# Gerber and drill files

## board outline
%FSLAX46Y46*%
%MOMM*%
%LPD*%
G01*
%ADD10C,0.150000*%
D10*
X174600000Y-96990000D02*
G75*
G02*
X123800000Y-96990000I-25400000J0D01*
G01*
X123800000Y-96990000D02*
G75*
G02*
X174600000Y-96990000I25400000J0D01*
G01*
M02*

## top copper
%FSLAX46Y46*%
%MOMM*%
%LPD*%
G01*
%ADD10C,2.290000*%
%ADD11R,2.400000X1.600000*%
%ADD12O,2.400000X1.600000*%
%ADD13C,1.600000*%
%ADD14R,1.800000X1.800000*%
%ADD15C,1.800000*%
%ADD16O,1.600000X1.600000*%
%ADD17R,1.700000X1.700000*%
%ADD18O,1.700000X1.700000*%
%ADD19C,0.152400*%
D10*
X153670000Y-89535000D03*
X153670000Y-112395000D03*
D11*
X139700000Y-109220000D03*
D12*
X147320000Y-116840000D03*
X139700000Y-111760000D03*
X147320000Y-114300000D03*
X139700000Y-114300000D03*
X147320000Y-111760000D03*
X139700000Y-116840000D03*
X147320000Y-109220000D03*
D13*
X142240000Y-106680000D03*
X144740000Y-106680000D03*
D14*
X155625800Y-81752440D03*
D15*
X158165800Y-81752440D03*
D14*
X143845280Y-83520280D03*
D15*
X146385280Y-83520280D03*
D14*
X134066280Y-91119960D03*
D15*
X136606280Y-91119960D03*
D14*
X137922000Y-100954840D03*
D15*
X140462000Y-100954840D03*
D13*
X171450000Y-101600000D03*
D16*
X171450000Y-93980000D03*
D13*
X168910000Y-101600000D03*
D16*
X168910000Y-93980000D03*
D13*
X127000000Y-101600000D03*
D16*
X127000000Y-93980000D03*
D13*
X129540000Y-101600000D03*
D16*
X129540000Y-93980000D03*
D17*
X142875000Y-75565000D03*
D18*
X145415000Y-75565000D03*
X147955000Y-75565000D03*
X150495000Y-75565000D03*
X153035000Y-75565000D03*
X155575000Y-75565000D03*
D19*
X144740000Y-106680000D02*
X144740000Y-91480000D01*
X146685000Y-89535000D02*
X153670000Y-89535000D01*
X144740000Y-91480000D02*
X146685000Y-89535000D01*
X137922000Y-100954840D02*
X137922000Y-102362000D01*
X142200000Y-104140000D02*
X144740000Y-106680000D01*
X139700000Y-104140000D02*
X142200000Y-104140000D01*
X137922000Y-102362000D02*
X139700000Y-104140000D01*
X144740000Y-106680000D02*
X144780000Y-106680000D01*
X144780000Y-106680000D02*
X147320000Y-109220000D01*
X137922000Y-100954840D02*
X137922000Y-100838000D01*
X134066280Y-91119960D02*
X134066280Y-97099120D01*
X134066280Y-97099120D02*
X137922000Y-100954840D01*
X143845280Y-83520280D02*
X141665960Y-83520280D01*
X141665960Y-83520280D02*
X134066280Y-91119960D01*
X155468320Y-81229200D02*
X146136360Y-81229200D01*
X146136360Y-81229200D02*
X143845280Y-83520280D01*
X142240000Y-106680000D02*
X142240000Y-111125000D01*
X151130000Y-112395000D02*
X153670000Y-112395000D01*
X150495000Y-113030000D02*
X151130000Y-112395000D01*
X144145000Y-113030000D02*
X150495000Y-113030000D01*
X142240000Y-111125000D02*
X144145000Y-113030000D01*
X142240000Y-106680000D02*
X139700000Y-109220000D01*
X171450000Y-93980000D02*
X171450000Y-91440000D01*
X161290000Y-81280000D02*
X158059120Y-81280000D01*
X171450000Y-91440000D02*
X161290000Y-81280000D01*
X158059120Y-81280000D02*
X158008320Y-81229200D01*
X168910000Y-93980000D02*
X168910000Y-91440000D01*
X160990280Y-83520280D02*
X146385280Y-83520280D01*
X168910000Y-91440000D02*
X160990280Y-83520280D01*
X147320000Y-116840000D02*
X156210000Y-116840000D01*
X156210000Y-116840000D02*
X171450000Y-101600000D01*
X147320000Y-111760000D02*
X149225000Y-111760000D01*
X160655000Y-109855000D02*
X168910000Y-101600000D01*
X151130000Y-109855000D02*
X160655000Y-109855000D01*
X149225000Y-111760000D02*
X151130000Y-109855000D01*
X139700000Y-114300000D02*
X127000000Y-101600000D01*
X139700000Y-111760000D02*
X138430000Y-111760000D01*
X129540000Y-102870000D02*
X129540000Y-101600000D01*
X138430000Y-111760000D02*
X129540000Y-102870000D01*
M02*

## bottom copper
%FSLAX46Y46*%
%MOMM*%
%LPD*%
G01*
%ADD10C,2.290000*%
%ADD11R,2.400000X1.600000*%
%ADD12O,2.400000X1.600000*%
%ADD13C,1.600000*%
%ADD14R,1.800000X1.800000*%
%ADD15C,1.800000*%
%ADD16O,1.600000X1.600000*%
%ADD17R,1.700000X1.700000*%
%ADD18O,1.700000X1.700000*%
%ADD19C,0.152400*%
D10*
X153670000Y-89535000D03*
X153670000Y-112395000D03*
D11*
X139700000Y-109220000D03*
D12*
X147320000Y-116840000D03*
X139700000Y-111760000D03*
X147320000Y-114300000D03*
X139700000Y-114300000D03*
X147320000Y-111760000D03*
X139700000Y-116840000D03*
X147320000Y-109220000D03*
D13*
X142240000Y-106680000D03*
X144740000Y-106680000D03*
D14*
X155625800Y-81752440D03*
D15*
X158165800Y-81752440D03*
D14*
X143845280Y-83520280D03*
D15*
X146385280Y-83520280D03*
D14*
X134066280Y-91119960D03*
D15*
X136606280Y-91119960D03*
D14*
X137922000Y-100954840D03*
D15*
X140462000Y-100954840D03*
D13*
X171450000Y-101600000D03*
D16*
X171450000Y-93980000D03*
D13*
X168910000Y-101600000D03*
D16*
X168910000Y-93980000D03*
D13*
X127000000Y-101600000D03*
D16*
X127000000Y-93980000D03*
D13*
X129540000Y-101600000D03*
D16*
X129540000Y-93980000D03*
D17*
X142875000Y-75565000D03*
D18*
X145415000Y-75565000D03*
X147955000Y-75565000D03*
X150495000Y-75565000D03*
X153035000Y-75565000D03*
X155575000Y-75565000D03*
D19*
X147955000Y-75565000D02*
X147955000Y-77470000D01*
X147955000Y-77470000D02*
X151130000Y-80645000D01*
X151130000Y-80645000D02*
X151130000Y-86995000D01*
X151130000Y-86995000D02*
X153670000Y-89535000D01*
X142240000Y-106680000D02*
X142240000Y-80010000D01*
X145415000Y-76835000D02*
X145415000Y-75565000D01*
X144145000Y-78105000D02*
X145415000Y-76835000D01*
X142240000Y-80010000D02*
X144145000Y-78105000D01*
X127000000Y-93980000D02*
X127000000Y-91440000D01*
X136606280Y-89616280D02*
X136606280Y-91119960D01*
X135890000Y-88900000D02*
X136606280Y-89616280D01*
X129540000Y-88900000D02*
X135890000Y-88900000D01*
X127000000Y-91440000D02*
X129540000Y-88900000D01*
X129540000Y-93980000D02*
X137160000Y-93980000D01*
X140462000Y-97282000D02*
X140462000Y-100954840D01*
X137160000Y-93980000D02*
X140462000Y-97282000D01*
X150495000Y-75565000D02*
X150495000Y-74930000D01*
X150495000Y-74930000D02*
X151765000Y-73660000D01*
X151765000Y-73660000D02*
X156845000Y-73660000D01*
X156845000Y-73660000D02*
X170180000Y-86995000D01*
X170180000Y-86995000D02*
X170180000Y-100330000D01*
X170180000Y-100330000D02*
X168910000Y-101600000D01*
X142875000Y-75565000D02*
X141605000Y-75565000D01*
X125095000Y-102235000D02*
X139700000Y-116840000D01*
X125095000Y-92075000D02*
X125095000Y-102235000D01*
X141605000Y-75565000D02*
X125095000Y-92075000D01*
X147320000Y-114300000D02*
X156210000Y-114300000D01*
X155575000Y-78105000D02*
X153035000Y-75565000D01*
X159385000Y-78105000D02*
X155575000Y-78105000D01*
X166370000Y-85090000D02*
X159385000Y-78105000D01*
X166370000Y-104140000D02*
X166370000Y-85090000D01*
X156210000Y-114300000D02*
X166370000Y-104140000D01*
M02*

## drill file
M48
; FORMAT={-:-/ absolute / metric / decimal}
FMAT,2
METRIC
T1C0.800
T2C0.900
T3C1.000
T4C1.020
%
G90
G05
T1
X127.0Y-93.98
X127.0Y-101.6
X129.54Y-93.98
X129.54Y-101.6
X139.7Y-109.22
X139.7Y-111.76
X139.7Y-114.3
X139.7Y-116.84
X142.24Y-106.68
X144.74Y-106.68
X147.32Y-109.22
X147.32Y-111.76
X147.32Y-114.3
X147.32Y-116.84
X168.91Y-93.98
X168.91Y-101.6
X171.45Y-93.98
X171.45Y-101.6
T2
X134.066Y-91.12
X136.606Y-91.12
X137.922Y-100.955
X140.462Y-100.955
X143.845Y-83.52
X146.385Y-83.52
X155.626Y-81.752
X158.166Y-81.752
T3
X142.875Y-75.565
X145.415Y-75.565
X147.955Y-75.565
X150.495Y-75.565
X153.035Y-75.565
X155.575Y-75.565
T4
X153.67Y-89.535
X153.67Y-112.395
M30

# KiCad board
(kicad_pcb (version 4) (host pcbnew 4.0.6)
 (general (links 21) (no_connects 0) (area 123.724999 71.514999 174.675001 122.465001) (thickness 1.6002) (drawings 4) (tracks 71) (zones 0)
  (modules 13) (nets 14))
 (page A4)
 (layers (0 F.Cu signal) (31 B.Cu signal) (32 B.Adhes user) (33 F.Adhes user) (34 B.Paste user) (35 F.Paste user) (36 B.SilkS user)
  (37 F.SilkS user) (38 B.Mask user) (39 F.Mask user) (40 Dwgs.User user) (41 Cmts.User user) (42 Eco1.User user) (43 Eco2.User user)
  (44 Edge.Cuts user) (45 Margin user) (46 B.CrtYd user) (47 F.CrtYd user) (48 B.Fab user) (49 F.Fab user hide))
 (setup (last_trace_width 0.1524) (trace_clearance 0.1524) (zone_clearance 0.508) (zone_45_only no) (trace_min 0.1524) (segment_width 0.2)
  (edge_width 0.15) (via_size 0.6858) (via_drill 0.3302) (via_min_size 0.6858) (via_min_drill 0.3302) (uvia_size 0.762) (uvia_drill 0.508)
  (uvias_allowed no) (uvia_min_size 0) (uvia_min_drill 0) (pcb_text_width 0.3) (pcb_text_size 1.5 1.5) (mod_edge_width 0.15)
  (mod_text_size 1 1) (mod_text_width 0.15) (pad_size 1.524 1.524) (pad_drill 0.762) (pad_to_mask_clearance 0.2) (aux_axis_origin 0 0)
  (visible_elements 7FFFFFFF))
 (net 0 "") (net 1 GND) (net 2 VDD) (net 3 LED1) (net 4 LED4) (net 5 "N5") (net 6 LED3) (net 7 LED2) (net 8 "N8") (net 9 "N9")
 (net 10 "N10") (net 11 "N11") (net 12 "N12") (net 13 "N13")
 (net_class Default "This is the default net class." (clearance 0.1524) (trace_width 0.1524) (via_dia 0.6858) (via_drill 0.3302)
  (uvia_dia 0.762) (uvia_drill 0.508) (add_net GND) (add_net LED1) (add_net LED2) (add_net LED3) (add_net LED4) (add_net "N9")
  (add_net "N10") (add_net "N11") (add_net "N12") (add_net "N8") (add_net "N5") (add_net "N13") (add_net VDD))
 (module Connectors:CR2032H (layer B.Cu) (at 153.67 112.395 270)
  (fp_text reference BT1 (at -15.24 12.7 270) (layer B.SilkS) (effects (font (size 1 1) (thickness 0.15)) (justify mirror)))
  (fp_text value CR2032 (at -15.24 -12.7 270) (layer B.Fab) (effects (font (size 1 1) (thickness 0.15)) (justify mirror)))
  (pad 2 thru_hole circle (at -22.86 0 270) (size 2.29 2.29) (drill 1.02) (layers *.Cu *.Mask) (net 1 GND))
  (pad 1 thru_hole circle (at 0 0 270) (size 2.29 2.29) (drill 1.02) (layers *.Cu *.Mask) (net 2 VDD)))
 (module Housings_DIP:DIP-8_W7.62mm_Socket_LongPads (layer F.Cu) (at 139.7 109.22)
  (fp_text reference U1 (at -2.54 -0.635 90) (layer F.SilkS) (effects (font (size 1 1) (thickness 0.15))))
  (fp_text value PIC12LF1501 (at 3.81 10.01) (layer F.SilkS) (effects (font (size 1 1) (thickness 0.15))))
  (pad 1 thru_hole rect (at 0 0) (size 2.4 1.6) (drill 0.8) (layers *.Cu *.Mask) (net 2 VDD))
  (pad 5 thru_hole oval (at 7.62 7.62) (size 2.4 1.6) (drill 0.8) (layers *.Cu *.Mask) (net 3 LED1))
  (pad 2 thru_hole oval (at 0 2.54) (size 2.4 1.6) (drill 0.8) (layers *.Cu *.Mask) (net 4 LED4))
  (pad 6 thru_hole oval (at 7.62 5.08) (size 2.4 1.6) (drill 0.8) (layers *.Cu *.Mask) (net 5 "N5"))
  (pad 3 thru_hole oval (at 0 5.08) (size 2.4 1.6) (drill 0.8) (layers *.Cu *.Mask) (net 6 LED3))
  (pad 7 thru_hole oval (at 7.62 2.54) (size 2.4 1.6) (drill 0.8) (layers *.Cu *.Mask) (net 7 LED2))
  (pad 4 thru_hole oval (at 0 7.62) (size 2.4 1.6) (drill 0.8) (layers *.Cu *.Mask) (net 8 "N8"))
  (pad 8 thru_hole oval (at 7.62 0) (size 2.4 1.6) (drill 0.8) (layers *.Cu *.Mask) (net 1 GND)))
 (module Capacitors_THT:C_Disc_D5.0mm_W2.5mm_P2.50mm (layer F.Cu) (at 142.24 106.68)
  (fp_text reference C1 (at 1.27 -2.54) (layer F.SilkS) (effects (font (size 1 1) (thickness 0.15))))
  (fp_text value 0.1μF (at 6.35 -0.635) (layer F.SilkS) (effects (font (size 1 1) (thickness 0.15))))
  (pad 1 thru_hole circle (at 0 0) (size 1.6 1.6) (drill 0.8) (layers *.Cu *.Mask) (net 2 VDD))
  (pad 2 thru_hole circle (at 2.5 0) (size 1.6 1.6) (drill 0.8) (layers *.Cu *.Mask) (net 1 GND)))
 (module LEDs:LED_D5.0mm (layer F.Cu) (at 155.6258 81.75244)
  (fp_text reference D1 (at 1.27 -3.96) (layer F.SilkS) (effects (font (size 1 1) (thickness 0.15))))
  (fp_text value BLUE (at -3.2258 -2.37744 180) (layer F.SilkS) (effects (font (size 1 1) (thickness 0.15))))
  (pad 1 thru_hole rect (at 0 0) (size 1.8 1.8) (drill 0.9) (layers *.Cu *.Mask) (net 1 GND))
  (pad 2 thru_hole circle (at 2.54 0) (size 1.8 1.8) (drill 0.9) (layers *.Cu *.Mask) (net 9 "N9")))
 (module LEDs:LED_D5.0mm (layer F.Cu) (at 143.84528 83.52028)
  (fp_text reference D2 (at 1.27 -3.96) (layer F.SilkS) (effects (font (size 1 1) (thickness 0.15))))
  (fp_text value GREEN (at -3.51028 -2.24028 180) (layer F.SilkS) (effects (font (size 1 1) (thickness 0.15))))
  (pad 1 thru_hole rect (at 0 0) (size 1.8 1.8) (drill 0.9) (layers *.Cu *.Mask) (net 1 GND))
  (pad 2 thru_hole circle (at 2.54 0) (size 1.8 1.8) (drill 0.9) (layers *.Cu *.Mask) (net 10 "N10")))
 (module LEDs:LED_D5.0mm (layer F.Cu) (at 134.06628 91.11996)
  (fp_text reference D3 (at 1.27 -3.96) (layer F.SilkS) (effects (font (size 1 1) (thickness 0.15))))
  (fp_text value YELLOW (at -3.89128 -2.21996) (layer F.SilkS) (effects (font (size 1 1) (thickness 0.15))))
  (pad 1 thru_hole rect (at 0 0) (size 1.8 1.8) (drill 0.9) (layers *.Cu *.Mask) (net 1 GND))
  (pad 2 thru_hole circle (at 2.54 0) (size 1.8 1.8) (drill 0.9) (layers *.Cu *.Mask) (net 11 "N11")))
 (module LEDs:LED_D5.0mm (layer F.Cu) (at 137.922 100.95484)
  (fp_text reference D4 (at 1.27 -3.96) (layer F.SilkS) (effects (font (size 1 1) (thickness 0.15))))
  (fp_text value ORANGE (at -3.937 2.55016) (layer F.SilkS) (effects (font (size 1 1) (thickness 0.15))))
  (pad 1 thru_hole rect (at 0 0) (size 1.8 1.8) (drill 0.9) (layers *.Cu *.Mask) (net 1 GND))
  (pad 2 thru_hole circle (at 2.54 0) (size 1.8 1.8) (drill 0.9) (layers *.Cu *.Mask) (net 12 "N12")))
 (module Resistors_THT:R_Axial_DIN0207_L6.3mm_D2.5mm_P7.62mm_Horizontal (layer F.Cu) (at 171.45 101.6 90)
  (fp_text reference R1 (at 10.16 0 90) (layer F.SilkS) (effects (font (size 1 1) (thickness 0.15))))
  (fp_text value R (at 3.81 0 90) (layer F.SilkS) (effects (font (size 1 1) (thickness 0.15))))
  (pad 1 thru_hole circle (at 0 0 90) (size 1.6 1.6) (drill 0.8) (layers *.Cu *.Mask) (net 3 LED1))
  (pad 2 thru_hole oval (at 7.62 0 90) (size 1.6 1.6) (drill 0.8) (layers *.Cu *.Mask) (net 9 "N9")))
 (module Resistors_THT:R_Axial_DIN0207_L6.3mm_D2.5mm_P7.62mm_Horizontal (layer F.Cu) (at 168.91 101.6 90)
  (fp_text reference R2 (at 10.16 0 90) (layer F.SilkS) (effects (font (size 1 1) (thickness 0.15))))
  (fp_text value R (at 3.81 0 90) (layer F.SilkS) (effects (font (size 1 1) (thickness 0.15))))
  (pad 1 thru_hole circle (at 0 0 90) (size 1.6 1.6) (drill 0.8) (layers *.Cu *.Mask) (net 7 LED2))
  (pad 2 thru_hole oval (at 7.62 0 90) (size 1.6 1.6) (drill 0.8) (layers *.Cu *.Mask) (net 10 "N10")))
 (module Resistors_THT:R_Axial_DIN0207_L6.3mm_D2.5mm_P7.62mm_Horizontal (layer F.Cu) (at 127 101.6 90)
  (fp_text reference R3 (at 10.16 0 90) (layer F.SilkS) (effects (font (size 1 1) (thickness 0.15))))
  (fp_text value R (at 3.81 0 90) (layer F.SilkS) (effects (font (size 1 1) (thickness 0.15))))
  (pad 1 thru_hole circle (at 0 0 90) (size 1.6 1.6) (drill 0.8) (layers *.Cu *.Mask) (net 6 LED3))
  (pad 2 thru_hole oval (at 7.62 0 90) (size 1.6 1.6) (drill 0.8) (layers *.Cu *.Mask) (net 11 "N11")))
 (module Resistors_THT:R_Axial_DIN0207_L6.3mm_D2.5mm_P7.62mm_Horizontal (layer F.Cu) (at 129.54 101.6 90)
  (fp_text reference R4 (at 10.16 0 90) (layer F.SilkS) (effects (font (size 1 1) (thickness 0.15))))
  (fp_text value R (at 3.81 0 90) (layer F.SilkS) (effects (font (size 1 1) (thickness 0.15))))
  (pad 1 thru_hole circle (at 0 0 90) (size 1.6 1.6) (drill 0.8) (layers *.Cu *.Mask) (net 4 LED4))
  (pad 2 thru_hole oval (at 7.62 0 90) (size 1.6 1.6) (drill 0.8) (layers *.Cu *.Mask) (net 12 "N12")))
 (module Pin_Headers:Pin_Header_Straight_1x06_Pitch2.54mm (layer F.Cu) (at 142.875 75.565 90)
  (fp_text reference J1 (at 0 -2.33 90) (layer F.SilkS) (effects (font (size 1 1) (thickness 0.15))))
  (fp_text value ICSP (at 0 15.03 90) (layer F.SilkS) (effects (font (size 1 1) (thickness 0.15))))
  (pad 1 thru_hole rect (at 0 0 90) (size 1.7 1.7) (drill 1) (layers *.Cu *.Mask) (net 8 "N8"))
  (pad 2 thru_hole oval (at 0 2.54 90) (size 1.7 1.7) (drill 1) (layers *.Cu *.Mask) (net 2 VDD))
  (pad 3 thru_hole oval (at 0 5.08 90) (size 1.7 1.7) (drill 1) (layers *.Cu *.Mask) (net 1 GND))
  (pad 4 thru_hole oval (at 0 7.62 90) (size 1.7 1.7) (drill 1) (layers *.Cu *.Mask) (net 7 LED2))
  (pad 5 thru_hole oval (at 0 10.16 90) (size 1.7 1.7) (drill 1) (layers *.Cu *.Mask) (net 5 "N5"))
  (pad 6 thru_hole oval (at 0 12.7 90) (size 1.7 1.7) (drill 1) (layers *.Cu *.Mask) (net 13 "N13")))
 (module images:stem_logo (layer F.Cu) (at 148.58492 92.53728)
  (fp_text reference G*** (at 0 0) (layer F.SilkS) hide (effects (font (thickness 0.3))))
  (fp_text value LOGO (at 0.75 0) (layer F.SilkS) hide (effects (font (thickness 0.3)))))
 (gr_circle (center 149.2 96.99) (end 174.6 96.99) (layer Edge.Cuts) (width 0.15))
 (segment (start 144.74 106.68) (end 144.74 91.48) (width 0.1524) (layer F.Cu) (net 1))
 (segment (start 146.685 89.535) (end 153.67 89.535) (width 0.1524) (layer F.Cu) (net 1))
 (segment (start 144.74 91.48) (end 146.685 89.535) (width 0.1524) (layer F.Cu) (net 1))
 (segment (start 147.955 75.565) (end 147.955 77.47) (width 0.1524) (layer B.Cu) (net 1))
 (segment (start 147.955 77.47) (end 151.13 80.645) (width 0.1524) (layer B.Cu) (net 1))
 (segment (start 151.13 80.645) (end 151.13 86.995) (width 0.1524) (layer B.Cu) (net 1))
 (segment (start 151.13 86.995) (end 153.67 89.535) (width 0.1524) (layer B.Cu) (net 1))
 (segment (start 137.922 100.95484) (end 137.922 102.362) (width 0.1524) (layer F.Cu) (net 1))
 (segment (start 142.2 104.14) (end 144.74 106.68) (width 0.1524) (layer F.Cu) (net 1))
 (segment (start 139.7 104.14) (end 142.2 104.14) (width 0.1524) (layer F.Cu) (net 1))
 (segment (start 137.922 102.362) (end 139.7 104.14) (width 0.1524) (layer F.Cu) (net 1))
 (segment (start 144.74 106.68) (end 144.78 106.68) (width 0.1524) (layer F.Cu) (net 1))
 (segment (start 144.78 106.68) (end 147.32 109.22) (width 0.1524) (layer F.Cu) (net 1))
 (segment (start 137.922 100.95484) (end 137.922 100.838) (width 0.1524) (layer F.Cu) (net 1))
 (segment (start 134.06628 91.11996) (end 134.06628 97.09912) (width 0.1524) (layer F.Cu) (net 1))
 (segment (start 134.06628 97.09912) (end 137.922 100.95484) (width 0.1524) (layer F.Cu) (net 1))
 (segment (start 143.84528 83.52028) (end 141.66596 83.52028) (width 0.1524) (layer F.Cu) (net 1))
 (segment (start 141.66596 83.52028) (end 134.06628 91.11996) (width 0.1524) (layer F.Cu) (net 1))
 (segment (start 155.46832 81.2292) (end 146.13636 81.2292) (width 0.1524) (layer F.Cu) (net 1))
 (segment (start 146.13636 81.2292) (end 143.84528 83.52028) (width 0.1524) (layer F.Cu) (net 1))
 (segment (start 142.24 106.68) (end 142.24 111.125) (width 0.1524) (layer F.Cu) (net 2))
 (segment (start 151.13 112.395) (end 153.67 112.395) (width 0.1524) (layer F.Cu) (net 2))
 (segment (start 150.495 113.03) (end 151.13 112.395) (width 0.1524) (layer F.Cu) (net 2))
 (segment (start 144.145 113.03) (end 150.495 113.03) (width 0.1524) (layer F.Cu) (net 2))
 (segment (start 142.24 111.125) (end 144.145 113.03) (width 0.1524) (layer F.Cu) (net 2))
 (segment (start 142.24 106.68) (end 142.24 80.01) (width 0.1524) (layer B.Cu) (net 2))
 (segment (start 145.415 76.835) (end 145.415 75.565) (width 0.1524) (layer B.Cu) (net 2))
 (segment (start 144.145 78.105) (end 145.415 76.835) (width 0.1524) (layer B.Cu) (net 2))
 (segment (start 142.24 80.01) (end 144.145 78.105) (width 0.1524) (layer B.Cu) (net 2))
 (segment (start 142.24 106.68) (end 139.7 109.22) (width 0.1524) (layer F.Cu) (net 2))
 (segment (start 171.45 93.98) (end 171.45 91.44) (width 0.1524) (layer F.Cu) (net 9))
 (segment (start 161.29 81.28) (end 158.05912 81.28) (width 0.1524) (layer F.Cu) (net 9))
 (segment (start 171.45 91.44) (end 161.29 81.28) (width 0.1524) (layer F.Cu) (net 9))
 (segment (start 158.05912 81.28) (end 158.00832 81.2292) (width 0.1524) (layer F.Cu) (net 9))
 (segment (start 168.91 93.98) (end 168.91 91.44) (width 0.1524) (layer F.Cu) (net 10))
 (segment (start 160.99028 83.52028) (end 146.38528 83.52028) (width 0.1524) (layer F.Cu) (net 10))
 (segment (start 168.91 91.44) (end 160.99028 83.52028) (width 0.1524) (layer F.Cu) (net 10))
 (segment (start 127 93.98) (end 127 91.44) (width 0.1524) (layer B.Cu) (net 11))
 (segment (start 136.60628 89.61628) (end 136.60628 91.11996) (width 0.1524) (layer B.Cu) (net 11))
 (segment (start 135.89 88.9) (end 136.60628 89.61628) (width 0.1524) (layer B.Cu) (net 11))
 (segment (start 129.54 88.9) (end 135.89 88.9) (width 0.1524) (layer B.Cu) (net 11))
 (segment (start 127 91.44) (end 129.54 88.9) (width 0.1524) (layer B.Cu) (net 11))
 (segment (start 129.54 93.98) (end 137.16 93.98) (width 0.1524) (layer B.Cu) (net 12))
 (segment (start 140.462 97.282) (end 140.462 100.95484) (width 0.1524) (layer B.Cu) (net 12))
 (segment (start 137.16 93.98) (end 140.462 97.282) (width 0.1524) (layer B.Cu) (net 12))
 (segment (start 147.32 116.84) (end 156.21 116.84) (width 0.1524) (layer F.Cu) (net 3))
 (segment (start 156.21 116.84) (end 171.45 101.6) (width 0.1524) (layer F.Cu) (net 3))
 (segment (start 150.495 75.565) (end 150.495 74.93) (width 0.1524) (layer B.Cu) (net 7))
 (segment (start 150.495 74.93) (end 151.765 73.66) (width 0.1524) (layer B.Cu) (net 7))
 (segment (start 151.765 73.66) (end 156.845 73.66) (width 0.1524) (layer B.Cu) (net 7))
 (segment (start 156.845 73.66) (end 170.18 86.995) (width 0.1524) (layer B.Cu) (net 7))
 (segment (start 170.18 86.995) (end 170.18 100.33) (width 0.1524) (layer B.Cu) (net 7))
 (segment (start 170.18 100.33) (end 168.91 101.6) (width 0.1524) (layer B.Cu) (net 7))
 (segment (start 147.32 111.76) (end 149.225 111.76) (width 0.1524) (layer F.Cu) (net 7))
 (segment (start 160.655 109.855) (end 168.91 101.6) (width 0.1524) (layer F.Cu) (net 7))
 (segment (start 151.13 109.855) (end 160.655 109.855) (width 0.1524) (layer F.Cu) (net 7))
 (segment (start 149.225 111.76) (end 151.13 109.855) (width 0.1524) (layer F.Cu) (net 7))
 (segment (start 139.7 114.3) (end 127 101.6) (width 0.1524) (layer F.Cu) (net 6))
 (segment (start 139.7 111.76) (end 138.43 111.76) (width 0.1524) (layer F.Cu) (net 4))
 (segment (start 129.54 102.87) (end 129.54 101.6) (width 0.1524) (layer F.Cu) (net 4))
 (segment (start 138.43 111.76) (end 129.54 102.87) (width 0.1524) (layer F.Cu) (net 4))
 (segment (start 142.875 75.565) (end 141.605 75.565) (width 0.1524) (layer B.Cu) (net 8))
 (segment (start 125.095 102.235) (end 139.7 116.84) (width 0.1524) (layer B.Cu) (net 8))
 (segment (start 125.095 92.075) (end 125.095 102.235) (width 0.1524) (layer B.Cu) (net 8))
 (segment (start 141.605 75.565) (end 125.095 92.075) (width 0.1524) (layer B.Cu) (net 8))
 (segment (start 147.32 114.3) (end 156.21 114.3) (width 0.1524) (layer B.Cu) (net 5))
 (segment (start 155.575 78.105) (end 153.035 75.565) (width 0.1524) (layer B.Cu) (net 5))
 (segment (start 159.385 78.105) (end 155.575 78.105) (width 0.1524) (layer B.Cu) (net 5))
 (segment (start 166.37 85.09) (end 159.385 78.105) (width 0.1524) (layer B.Cu) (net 5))
 (segment (start 166.37 104.14) (end 166.37 85.09) (width 0.1524) (layer B.Cu) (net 5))
 (segment (start 156.21 114.3) (end 166.37 104.14) (width 0.1524) (layer B.Cu) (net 5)))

